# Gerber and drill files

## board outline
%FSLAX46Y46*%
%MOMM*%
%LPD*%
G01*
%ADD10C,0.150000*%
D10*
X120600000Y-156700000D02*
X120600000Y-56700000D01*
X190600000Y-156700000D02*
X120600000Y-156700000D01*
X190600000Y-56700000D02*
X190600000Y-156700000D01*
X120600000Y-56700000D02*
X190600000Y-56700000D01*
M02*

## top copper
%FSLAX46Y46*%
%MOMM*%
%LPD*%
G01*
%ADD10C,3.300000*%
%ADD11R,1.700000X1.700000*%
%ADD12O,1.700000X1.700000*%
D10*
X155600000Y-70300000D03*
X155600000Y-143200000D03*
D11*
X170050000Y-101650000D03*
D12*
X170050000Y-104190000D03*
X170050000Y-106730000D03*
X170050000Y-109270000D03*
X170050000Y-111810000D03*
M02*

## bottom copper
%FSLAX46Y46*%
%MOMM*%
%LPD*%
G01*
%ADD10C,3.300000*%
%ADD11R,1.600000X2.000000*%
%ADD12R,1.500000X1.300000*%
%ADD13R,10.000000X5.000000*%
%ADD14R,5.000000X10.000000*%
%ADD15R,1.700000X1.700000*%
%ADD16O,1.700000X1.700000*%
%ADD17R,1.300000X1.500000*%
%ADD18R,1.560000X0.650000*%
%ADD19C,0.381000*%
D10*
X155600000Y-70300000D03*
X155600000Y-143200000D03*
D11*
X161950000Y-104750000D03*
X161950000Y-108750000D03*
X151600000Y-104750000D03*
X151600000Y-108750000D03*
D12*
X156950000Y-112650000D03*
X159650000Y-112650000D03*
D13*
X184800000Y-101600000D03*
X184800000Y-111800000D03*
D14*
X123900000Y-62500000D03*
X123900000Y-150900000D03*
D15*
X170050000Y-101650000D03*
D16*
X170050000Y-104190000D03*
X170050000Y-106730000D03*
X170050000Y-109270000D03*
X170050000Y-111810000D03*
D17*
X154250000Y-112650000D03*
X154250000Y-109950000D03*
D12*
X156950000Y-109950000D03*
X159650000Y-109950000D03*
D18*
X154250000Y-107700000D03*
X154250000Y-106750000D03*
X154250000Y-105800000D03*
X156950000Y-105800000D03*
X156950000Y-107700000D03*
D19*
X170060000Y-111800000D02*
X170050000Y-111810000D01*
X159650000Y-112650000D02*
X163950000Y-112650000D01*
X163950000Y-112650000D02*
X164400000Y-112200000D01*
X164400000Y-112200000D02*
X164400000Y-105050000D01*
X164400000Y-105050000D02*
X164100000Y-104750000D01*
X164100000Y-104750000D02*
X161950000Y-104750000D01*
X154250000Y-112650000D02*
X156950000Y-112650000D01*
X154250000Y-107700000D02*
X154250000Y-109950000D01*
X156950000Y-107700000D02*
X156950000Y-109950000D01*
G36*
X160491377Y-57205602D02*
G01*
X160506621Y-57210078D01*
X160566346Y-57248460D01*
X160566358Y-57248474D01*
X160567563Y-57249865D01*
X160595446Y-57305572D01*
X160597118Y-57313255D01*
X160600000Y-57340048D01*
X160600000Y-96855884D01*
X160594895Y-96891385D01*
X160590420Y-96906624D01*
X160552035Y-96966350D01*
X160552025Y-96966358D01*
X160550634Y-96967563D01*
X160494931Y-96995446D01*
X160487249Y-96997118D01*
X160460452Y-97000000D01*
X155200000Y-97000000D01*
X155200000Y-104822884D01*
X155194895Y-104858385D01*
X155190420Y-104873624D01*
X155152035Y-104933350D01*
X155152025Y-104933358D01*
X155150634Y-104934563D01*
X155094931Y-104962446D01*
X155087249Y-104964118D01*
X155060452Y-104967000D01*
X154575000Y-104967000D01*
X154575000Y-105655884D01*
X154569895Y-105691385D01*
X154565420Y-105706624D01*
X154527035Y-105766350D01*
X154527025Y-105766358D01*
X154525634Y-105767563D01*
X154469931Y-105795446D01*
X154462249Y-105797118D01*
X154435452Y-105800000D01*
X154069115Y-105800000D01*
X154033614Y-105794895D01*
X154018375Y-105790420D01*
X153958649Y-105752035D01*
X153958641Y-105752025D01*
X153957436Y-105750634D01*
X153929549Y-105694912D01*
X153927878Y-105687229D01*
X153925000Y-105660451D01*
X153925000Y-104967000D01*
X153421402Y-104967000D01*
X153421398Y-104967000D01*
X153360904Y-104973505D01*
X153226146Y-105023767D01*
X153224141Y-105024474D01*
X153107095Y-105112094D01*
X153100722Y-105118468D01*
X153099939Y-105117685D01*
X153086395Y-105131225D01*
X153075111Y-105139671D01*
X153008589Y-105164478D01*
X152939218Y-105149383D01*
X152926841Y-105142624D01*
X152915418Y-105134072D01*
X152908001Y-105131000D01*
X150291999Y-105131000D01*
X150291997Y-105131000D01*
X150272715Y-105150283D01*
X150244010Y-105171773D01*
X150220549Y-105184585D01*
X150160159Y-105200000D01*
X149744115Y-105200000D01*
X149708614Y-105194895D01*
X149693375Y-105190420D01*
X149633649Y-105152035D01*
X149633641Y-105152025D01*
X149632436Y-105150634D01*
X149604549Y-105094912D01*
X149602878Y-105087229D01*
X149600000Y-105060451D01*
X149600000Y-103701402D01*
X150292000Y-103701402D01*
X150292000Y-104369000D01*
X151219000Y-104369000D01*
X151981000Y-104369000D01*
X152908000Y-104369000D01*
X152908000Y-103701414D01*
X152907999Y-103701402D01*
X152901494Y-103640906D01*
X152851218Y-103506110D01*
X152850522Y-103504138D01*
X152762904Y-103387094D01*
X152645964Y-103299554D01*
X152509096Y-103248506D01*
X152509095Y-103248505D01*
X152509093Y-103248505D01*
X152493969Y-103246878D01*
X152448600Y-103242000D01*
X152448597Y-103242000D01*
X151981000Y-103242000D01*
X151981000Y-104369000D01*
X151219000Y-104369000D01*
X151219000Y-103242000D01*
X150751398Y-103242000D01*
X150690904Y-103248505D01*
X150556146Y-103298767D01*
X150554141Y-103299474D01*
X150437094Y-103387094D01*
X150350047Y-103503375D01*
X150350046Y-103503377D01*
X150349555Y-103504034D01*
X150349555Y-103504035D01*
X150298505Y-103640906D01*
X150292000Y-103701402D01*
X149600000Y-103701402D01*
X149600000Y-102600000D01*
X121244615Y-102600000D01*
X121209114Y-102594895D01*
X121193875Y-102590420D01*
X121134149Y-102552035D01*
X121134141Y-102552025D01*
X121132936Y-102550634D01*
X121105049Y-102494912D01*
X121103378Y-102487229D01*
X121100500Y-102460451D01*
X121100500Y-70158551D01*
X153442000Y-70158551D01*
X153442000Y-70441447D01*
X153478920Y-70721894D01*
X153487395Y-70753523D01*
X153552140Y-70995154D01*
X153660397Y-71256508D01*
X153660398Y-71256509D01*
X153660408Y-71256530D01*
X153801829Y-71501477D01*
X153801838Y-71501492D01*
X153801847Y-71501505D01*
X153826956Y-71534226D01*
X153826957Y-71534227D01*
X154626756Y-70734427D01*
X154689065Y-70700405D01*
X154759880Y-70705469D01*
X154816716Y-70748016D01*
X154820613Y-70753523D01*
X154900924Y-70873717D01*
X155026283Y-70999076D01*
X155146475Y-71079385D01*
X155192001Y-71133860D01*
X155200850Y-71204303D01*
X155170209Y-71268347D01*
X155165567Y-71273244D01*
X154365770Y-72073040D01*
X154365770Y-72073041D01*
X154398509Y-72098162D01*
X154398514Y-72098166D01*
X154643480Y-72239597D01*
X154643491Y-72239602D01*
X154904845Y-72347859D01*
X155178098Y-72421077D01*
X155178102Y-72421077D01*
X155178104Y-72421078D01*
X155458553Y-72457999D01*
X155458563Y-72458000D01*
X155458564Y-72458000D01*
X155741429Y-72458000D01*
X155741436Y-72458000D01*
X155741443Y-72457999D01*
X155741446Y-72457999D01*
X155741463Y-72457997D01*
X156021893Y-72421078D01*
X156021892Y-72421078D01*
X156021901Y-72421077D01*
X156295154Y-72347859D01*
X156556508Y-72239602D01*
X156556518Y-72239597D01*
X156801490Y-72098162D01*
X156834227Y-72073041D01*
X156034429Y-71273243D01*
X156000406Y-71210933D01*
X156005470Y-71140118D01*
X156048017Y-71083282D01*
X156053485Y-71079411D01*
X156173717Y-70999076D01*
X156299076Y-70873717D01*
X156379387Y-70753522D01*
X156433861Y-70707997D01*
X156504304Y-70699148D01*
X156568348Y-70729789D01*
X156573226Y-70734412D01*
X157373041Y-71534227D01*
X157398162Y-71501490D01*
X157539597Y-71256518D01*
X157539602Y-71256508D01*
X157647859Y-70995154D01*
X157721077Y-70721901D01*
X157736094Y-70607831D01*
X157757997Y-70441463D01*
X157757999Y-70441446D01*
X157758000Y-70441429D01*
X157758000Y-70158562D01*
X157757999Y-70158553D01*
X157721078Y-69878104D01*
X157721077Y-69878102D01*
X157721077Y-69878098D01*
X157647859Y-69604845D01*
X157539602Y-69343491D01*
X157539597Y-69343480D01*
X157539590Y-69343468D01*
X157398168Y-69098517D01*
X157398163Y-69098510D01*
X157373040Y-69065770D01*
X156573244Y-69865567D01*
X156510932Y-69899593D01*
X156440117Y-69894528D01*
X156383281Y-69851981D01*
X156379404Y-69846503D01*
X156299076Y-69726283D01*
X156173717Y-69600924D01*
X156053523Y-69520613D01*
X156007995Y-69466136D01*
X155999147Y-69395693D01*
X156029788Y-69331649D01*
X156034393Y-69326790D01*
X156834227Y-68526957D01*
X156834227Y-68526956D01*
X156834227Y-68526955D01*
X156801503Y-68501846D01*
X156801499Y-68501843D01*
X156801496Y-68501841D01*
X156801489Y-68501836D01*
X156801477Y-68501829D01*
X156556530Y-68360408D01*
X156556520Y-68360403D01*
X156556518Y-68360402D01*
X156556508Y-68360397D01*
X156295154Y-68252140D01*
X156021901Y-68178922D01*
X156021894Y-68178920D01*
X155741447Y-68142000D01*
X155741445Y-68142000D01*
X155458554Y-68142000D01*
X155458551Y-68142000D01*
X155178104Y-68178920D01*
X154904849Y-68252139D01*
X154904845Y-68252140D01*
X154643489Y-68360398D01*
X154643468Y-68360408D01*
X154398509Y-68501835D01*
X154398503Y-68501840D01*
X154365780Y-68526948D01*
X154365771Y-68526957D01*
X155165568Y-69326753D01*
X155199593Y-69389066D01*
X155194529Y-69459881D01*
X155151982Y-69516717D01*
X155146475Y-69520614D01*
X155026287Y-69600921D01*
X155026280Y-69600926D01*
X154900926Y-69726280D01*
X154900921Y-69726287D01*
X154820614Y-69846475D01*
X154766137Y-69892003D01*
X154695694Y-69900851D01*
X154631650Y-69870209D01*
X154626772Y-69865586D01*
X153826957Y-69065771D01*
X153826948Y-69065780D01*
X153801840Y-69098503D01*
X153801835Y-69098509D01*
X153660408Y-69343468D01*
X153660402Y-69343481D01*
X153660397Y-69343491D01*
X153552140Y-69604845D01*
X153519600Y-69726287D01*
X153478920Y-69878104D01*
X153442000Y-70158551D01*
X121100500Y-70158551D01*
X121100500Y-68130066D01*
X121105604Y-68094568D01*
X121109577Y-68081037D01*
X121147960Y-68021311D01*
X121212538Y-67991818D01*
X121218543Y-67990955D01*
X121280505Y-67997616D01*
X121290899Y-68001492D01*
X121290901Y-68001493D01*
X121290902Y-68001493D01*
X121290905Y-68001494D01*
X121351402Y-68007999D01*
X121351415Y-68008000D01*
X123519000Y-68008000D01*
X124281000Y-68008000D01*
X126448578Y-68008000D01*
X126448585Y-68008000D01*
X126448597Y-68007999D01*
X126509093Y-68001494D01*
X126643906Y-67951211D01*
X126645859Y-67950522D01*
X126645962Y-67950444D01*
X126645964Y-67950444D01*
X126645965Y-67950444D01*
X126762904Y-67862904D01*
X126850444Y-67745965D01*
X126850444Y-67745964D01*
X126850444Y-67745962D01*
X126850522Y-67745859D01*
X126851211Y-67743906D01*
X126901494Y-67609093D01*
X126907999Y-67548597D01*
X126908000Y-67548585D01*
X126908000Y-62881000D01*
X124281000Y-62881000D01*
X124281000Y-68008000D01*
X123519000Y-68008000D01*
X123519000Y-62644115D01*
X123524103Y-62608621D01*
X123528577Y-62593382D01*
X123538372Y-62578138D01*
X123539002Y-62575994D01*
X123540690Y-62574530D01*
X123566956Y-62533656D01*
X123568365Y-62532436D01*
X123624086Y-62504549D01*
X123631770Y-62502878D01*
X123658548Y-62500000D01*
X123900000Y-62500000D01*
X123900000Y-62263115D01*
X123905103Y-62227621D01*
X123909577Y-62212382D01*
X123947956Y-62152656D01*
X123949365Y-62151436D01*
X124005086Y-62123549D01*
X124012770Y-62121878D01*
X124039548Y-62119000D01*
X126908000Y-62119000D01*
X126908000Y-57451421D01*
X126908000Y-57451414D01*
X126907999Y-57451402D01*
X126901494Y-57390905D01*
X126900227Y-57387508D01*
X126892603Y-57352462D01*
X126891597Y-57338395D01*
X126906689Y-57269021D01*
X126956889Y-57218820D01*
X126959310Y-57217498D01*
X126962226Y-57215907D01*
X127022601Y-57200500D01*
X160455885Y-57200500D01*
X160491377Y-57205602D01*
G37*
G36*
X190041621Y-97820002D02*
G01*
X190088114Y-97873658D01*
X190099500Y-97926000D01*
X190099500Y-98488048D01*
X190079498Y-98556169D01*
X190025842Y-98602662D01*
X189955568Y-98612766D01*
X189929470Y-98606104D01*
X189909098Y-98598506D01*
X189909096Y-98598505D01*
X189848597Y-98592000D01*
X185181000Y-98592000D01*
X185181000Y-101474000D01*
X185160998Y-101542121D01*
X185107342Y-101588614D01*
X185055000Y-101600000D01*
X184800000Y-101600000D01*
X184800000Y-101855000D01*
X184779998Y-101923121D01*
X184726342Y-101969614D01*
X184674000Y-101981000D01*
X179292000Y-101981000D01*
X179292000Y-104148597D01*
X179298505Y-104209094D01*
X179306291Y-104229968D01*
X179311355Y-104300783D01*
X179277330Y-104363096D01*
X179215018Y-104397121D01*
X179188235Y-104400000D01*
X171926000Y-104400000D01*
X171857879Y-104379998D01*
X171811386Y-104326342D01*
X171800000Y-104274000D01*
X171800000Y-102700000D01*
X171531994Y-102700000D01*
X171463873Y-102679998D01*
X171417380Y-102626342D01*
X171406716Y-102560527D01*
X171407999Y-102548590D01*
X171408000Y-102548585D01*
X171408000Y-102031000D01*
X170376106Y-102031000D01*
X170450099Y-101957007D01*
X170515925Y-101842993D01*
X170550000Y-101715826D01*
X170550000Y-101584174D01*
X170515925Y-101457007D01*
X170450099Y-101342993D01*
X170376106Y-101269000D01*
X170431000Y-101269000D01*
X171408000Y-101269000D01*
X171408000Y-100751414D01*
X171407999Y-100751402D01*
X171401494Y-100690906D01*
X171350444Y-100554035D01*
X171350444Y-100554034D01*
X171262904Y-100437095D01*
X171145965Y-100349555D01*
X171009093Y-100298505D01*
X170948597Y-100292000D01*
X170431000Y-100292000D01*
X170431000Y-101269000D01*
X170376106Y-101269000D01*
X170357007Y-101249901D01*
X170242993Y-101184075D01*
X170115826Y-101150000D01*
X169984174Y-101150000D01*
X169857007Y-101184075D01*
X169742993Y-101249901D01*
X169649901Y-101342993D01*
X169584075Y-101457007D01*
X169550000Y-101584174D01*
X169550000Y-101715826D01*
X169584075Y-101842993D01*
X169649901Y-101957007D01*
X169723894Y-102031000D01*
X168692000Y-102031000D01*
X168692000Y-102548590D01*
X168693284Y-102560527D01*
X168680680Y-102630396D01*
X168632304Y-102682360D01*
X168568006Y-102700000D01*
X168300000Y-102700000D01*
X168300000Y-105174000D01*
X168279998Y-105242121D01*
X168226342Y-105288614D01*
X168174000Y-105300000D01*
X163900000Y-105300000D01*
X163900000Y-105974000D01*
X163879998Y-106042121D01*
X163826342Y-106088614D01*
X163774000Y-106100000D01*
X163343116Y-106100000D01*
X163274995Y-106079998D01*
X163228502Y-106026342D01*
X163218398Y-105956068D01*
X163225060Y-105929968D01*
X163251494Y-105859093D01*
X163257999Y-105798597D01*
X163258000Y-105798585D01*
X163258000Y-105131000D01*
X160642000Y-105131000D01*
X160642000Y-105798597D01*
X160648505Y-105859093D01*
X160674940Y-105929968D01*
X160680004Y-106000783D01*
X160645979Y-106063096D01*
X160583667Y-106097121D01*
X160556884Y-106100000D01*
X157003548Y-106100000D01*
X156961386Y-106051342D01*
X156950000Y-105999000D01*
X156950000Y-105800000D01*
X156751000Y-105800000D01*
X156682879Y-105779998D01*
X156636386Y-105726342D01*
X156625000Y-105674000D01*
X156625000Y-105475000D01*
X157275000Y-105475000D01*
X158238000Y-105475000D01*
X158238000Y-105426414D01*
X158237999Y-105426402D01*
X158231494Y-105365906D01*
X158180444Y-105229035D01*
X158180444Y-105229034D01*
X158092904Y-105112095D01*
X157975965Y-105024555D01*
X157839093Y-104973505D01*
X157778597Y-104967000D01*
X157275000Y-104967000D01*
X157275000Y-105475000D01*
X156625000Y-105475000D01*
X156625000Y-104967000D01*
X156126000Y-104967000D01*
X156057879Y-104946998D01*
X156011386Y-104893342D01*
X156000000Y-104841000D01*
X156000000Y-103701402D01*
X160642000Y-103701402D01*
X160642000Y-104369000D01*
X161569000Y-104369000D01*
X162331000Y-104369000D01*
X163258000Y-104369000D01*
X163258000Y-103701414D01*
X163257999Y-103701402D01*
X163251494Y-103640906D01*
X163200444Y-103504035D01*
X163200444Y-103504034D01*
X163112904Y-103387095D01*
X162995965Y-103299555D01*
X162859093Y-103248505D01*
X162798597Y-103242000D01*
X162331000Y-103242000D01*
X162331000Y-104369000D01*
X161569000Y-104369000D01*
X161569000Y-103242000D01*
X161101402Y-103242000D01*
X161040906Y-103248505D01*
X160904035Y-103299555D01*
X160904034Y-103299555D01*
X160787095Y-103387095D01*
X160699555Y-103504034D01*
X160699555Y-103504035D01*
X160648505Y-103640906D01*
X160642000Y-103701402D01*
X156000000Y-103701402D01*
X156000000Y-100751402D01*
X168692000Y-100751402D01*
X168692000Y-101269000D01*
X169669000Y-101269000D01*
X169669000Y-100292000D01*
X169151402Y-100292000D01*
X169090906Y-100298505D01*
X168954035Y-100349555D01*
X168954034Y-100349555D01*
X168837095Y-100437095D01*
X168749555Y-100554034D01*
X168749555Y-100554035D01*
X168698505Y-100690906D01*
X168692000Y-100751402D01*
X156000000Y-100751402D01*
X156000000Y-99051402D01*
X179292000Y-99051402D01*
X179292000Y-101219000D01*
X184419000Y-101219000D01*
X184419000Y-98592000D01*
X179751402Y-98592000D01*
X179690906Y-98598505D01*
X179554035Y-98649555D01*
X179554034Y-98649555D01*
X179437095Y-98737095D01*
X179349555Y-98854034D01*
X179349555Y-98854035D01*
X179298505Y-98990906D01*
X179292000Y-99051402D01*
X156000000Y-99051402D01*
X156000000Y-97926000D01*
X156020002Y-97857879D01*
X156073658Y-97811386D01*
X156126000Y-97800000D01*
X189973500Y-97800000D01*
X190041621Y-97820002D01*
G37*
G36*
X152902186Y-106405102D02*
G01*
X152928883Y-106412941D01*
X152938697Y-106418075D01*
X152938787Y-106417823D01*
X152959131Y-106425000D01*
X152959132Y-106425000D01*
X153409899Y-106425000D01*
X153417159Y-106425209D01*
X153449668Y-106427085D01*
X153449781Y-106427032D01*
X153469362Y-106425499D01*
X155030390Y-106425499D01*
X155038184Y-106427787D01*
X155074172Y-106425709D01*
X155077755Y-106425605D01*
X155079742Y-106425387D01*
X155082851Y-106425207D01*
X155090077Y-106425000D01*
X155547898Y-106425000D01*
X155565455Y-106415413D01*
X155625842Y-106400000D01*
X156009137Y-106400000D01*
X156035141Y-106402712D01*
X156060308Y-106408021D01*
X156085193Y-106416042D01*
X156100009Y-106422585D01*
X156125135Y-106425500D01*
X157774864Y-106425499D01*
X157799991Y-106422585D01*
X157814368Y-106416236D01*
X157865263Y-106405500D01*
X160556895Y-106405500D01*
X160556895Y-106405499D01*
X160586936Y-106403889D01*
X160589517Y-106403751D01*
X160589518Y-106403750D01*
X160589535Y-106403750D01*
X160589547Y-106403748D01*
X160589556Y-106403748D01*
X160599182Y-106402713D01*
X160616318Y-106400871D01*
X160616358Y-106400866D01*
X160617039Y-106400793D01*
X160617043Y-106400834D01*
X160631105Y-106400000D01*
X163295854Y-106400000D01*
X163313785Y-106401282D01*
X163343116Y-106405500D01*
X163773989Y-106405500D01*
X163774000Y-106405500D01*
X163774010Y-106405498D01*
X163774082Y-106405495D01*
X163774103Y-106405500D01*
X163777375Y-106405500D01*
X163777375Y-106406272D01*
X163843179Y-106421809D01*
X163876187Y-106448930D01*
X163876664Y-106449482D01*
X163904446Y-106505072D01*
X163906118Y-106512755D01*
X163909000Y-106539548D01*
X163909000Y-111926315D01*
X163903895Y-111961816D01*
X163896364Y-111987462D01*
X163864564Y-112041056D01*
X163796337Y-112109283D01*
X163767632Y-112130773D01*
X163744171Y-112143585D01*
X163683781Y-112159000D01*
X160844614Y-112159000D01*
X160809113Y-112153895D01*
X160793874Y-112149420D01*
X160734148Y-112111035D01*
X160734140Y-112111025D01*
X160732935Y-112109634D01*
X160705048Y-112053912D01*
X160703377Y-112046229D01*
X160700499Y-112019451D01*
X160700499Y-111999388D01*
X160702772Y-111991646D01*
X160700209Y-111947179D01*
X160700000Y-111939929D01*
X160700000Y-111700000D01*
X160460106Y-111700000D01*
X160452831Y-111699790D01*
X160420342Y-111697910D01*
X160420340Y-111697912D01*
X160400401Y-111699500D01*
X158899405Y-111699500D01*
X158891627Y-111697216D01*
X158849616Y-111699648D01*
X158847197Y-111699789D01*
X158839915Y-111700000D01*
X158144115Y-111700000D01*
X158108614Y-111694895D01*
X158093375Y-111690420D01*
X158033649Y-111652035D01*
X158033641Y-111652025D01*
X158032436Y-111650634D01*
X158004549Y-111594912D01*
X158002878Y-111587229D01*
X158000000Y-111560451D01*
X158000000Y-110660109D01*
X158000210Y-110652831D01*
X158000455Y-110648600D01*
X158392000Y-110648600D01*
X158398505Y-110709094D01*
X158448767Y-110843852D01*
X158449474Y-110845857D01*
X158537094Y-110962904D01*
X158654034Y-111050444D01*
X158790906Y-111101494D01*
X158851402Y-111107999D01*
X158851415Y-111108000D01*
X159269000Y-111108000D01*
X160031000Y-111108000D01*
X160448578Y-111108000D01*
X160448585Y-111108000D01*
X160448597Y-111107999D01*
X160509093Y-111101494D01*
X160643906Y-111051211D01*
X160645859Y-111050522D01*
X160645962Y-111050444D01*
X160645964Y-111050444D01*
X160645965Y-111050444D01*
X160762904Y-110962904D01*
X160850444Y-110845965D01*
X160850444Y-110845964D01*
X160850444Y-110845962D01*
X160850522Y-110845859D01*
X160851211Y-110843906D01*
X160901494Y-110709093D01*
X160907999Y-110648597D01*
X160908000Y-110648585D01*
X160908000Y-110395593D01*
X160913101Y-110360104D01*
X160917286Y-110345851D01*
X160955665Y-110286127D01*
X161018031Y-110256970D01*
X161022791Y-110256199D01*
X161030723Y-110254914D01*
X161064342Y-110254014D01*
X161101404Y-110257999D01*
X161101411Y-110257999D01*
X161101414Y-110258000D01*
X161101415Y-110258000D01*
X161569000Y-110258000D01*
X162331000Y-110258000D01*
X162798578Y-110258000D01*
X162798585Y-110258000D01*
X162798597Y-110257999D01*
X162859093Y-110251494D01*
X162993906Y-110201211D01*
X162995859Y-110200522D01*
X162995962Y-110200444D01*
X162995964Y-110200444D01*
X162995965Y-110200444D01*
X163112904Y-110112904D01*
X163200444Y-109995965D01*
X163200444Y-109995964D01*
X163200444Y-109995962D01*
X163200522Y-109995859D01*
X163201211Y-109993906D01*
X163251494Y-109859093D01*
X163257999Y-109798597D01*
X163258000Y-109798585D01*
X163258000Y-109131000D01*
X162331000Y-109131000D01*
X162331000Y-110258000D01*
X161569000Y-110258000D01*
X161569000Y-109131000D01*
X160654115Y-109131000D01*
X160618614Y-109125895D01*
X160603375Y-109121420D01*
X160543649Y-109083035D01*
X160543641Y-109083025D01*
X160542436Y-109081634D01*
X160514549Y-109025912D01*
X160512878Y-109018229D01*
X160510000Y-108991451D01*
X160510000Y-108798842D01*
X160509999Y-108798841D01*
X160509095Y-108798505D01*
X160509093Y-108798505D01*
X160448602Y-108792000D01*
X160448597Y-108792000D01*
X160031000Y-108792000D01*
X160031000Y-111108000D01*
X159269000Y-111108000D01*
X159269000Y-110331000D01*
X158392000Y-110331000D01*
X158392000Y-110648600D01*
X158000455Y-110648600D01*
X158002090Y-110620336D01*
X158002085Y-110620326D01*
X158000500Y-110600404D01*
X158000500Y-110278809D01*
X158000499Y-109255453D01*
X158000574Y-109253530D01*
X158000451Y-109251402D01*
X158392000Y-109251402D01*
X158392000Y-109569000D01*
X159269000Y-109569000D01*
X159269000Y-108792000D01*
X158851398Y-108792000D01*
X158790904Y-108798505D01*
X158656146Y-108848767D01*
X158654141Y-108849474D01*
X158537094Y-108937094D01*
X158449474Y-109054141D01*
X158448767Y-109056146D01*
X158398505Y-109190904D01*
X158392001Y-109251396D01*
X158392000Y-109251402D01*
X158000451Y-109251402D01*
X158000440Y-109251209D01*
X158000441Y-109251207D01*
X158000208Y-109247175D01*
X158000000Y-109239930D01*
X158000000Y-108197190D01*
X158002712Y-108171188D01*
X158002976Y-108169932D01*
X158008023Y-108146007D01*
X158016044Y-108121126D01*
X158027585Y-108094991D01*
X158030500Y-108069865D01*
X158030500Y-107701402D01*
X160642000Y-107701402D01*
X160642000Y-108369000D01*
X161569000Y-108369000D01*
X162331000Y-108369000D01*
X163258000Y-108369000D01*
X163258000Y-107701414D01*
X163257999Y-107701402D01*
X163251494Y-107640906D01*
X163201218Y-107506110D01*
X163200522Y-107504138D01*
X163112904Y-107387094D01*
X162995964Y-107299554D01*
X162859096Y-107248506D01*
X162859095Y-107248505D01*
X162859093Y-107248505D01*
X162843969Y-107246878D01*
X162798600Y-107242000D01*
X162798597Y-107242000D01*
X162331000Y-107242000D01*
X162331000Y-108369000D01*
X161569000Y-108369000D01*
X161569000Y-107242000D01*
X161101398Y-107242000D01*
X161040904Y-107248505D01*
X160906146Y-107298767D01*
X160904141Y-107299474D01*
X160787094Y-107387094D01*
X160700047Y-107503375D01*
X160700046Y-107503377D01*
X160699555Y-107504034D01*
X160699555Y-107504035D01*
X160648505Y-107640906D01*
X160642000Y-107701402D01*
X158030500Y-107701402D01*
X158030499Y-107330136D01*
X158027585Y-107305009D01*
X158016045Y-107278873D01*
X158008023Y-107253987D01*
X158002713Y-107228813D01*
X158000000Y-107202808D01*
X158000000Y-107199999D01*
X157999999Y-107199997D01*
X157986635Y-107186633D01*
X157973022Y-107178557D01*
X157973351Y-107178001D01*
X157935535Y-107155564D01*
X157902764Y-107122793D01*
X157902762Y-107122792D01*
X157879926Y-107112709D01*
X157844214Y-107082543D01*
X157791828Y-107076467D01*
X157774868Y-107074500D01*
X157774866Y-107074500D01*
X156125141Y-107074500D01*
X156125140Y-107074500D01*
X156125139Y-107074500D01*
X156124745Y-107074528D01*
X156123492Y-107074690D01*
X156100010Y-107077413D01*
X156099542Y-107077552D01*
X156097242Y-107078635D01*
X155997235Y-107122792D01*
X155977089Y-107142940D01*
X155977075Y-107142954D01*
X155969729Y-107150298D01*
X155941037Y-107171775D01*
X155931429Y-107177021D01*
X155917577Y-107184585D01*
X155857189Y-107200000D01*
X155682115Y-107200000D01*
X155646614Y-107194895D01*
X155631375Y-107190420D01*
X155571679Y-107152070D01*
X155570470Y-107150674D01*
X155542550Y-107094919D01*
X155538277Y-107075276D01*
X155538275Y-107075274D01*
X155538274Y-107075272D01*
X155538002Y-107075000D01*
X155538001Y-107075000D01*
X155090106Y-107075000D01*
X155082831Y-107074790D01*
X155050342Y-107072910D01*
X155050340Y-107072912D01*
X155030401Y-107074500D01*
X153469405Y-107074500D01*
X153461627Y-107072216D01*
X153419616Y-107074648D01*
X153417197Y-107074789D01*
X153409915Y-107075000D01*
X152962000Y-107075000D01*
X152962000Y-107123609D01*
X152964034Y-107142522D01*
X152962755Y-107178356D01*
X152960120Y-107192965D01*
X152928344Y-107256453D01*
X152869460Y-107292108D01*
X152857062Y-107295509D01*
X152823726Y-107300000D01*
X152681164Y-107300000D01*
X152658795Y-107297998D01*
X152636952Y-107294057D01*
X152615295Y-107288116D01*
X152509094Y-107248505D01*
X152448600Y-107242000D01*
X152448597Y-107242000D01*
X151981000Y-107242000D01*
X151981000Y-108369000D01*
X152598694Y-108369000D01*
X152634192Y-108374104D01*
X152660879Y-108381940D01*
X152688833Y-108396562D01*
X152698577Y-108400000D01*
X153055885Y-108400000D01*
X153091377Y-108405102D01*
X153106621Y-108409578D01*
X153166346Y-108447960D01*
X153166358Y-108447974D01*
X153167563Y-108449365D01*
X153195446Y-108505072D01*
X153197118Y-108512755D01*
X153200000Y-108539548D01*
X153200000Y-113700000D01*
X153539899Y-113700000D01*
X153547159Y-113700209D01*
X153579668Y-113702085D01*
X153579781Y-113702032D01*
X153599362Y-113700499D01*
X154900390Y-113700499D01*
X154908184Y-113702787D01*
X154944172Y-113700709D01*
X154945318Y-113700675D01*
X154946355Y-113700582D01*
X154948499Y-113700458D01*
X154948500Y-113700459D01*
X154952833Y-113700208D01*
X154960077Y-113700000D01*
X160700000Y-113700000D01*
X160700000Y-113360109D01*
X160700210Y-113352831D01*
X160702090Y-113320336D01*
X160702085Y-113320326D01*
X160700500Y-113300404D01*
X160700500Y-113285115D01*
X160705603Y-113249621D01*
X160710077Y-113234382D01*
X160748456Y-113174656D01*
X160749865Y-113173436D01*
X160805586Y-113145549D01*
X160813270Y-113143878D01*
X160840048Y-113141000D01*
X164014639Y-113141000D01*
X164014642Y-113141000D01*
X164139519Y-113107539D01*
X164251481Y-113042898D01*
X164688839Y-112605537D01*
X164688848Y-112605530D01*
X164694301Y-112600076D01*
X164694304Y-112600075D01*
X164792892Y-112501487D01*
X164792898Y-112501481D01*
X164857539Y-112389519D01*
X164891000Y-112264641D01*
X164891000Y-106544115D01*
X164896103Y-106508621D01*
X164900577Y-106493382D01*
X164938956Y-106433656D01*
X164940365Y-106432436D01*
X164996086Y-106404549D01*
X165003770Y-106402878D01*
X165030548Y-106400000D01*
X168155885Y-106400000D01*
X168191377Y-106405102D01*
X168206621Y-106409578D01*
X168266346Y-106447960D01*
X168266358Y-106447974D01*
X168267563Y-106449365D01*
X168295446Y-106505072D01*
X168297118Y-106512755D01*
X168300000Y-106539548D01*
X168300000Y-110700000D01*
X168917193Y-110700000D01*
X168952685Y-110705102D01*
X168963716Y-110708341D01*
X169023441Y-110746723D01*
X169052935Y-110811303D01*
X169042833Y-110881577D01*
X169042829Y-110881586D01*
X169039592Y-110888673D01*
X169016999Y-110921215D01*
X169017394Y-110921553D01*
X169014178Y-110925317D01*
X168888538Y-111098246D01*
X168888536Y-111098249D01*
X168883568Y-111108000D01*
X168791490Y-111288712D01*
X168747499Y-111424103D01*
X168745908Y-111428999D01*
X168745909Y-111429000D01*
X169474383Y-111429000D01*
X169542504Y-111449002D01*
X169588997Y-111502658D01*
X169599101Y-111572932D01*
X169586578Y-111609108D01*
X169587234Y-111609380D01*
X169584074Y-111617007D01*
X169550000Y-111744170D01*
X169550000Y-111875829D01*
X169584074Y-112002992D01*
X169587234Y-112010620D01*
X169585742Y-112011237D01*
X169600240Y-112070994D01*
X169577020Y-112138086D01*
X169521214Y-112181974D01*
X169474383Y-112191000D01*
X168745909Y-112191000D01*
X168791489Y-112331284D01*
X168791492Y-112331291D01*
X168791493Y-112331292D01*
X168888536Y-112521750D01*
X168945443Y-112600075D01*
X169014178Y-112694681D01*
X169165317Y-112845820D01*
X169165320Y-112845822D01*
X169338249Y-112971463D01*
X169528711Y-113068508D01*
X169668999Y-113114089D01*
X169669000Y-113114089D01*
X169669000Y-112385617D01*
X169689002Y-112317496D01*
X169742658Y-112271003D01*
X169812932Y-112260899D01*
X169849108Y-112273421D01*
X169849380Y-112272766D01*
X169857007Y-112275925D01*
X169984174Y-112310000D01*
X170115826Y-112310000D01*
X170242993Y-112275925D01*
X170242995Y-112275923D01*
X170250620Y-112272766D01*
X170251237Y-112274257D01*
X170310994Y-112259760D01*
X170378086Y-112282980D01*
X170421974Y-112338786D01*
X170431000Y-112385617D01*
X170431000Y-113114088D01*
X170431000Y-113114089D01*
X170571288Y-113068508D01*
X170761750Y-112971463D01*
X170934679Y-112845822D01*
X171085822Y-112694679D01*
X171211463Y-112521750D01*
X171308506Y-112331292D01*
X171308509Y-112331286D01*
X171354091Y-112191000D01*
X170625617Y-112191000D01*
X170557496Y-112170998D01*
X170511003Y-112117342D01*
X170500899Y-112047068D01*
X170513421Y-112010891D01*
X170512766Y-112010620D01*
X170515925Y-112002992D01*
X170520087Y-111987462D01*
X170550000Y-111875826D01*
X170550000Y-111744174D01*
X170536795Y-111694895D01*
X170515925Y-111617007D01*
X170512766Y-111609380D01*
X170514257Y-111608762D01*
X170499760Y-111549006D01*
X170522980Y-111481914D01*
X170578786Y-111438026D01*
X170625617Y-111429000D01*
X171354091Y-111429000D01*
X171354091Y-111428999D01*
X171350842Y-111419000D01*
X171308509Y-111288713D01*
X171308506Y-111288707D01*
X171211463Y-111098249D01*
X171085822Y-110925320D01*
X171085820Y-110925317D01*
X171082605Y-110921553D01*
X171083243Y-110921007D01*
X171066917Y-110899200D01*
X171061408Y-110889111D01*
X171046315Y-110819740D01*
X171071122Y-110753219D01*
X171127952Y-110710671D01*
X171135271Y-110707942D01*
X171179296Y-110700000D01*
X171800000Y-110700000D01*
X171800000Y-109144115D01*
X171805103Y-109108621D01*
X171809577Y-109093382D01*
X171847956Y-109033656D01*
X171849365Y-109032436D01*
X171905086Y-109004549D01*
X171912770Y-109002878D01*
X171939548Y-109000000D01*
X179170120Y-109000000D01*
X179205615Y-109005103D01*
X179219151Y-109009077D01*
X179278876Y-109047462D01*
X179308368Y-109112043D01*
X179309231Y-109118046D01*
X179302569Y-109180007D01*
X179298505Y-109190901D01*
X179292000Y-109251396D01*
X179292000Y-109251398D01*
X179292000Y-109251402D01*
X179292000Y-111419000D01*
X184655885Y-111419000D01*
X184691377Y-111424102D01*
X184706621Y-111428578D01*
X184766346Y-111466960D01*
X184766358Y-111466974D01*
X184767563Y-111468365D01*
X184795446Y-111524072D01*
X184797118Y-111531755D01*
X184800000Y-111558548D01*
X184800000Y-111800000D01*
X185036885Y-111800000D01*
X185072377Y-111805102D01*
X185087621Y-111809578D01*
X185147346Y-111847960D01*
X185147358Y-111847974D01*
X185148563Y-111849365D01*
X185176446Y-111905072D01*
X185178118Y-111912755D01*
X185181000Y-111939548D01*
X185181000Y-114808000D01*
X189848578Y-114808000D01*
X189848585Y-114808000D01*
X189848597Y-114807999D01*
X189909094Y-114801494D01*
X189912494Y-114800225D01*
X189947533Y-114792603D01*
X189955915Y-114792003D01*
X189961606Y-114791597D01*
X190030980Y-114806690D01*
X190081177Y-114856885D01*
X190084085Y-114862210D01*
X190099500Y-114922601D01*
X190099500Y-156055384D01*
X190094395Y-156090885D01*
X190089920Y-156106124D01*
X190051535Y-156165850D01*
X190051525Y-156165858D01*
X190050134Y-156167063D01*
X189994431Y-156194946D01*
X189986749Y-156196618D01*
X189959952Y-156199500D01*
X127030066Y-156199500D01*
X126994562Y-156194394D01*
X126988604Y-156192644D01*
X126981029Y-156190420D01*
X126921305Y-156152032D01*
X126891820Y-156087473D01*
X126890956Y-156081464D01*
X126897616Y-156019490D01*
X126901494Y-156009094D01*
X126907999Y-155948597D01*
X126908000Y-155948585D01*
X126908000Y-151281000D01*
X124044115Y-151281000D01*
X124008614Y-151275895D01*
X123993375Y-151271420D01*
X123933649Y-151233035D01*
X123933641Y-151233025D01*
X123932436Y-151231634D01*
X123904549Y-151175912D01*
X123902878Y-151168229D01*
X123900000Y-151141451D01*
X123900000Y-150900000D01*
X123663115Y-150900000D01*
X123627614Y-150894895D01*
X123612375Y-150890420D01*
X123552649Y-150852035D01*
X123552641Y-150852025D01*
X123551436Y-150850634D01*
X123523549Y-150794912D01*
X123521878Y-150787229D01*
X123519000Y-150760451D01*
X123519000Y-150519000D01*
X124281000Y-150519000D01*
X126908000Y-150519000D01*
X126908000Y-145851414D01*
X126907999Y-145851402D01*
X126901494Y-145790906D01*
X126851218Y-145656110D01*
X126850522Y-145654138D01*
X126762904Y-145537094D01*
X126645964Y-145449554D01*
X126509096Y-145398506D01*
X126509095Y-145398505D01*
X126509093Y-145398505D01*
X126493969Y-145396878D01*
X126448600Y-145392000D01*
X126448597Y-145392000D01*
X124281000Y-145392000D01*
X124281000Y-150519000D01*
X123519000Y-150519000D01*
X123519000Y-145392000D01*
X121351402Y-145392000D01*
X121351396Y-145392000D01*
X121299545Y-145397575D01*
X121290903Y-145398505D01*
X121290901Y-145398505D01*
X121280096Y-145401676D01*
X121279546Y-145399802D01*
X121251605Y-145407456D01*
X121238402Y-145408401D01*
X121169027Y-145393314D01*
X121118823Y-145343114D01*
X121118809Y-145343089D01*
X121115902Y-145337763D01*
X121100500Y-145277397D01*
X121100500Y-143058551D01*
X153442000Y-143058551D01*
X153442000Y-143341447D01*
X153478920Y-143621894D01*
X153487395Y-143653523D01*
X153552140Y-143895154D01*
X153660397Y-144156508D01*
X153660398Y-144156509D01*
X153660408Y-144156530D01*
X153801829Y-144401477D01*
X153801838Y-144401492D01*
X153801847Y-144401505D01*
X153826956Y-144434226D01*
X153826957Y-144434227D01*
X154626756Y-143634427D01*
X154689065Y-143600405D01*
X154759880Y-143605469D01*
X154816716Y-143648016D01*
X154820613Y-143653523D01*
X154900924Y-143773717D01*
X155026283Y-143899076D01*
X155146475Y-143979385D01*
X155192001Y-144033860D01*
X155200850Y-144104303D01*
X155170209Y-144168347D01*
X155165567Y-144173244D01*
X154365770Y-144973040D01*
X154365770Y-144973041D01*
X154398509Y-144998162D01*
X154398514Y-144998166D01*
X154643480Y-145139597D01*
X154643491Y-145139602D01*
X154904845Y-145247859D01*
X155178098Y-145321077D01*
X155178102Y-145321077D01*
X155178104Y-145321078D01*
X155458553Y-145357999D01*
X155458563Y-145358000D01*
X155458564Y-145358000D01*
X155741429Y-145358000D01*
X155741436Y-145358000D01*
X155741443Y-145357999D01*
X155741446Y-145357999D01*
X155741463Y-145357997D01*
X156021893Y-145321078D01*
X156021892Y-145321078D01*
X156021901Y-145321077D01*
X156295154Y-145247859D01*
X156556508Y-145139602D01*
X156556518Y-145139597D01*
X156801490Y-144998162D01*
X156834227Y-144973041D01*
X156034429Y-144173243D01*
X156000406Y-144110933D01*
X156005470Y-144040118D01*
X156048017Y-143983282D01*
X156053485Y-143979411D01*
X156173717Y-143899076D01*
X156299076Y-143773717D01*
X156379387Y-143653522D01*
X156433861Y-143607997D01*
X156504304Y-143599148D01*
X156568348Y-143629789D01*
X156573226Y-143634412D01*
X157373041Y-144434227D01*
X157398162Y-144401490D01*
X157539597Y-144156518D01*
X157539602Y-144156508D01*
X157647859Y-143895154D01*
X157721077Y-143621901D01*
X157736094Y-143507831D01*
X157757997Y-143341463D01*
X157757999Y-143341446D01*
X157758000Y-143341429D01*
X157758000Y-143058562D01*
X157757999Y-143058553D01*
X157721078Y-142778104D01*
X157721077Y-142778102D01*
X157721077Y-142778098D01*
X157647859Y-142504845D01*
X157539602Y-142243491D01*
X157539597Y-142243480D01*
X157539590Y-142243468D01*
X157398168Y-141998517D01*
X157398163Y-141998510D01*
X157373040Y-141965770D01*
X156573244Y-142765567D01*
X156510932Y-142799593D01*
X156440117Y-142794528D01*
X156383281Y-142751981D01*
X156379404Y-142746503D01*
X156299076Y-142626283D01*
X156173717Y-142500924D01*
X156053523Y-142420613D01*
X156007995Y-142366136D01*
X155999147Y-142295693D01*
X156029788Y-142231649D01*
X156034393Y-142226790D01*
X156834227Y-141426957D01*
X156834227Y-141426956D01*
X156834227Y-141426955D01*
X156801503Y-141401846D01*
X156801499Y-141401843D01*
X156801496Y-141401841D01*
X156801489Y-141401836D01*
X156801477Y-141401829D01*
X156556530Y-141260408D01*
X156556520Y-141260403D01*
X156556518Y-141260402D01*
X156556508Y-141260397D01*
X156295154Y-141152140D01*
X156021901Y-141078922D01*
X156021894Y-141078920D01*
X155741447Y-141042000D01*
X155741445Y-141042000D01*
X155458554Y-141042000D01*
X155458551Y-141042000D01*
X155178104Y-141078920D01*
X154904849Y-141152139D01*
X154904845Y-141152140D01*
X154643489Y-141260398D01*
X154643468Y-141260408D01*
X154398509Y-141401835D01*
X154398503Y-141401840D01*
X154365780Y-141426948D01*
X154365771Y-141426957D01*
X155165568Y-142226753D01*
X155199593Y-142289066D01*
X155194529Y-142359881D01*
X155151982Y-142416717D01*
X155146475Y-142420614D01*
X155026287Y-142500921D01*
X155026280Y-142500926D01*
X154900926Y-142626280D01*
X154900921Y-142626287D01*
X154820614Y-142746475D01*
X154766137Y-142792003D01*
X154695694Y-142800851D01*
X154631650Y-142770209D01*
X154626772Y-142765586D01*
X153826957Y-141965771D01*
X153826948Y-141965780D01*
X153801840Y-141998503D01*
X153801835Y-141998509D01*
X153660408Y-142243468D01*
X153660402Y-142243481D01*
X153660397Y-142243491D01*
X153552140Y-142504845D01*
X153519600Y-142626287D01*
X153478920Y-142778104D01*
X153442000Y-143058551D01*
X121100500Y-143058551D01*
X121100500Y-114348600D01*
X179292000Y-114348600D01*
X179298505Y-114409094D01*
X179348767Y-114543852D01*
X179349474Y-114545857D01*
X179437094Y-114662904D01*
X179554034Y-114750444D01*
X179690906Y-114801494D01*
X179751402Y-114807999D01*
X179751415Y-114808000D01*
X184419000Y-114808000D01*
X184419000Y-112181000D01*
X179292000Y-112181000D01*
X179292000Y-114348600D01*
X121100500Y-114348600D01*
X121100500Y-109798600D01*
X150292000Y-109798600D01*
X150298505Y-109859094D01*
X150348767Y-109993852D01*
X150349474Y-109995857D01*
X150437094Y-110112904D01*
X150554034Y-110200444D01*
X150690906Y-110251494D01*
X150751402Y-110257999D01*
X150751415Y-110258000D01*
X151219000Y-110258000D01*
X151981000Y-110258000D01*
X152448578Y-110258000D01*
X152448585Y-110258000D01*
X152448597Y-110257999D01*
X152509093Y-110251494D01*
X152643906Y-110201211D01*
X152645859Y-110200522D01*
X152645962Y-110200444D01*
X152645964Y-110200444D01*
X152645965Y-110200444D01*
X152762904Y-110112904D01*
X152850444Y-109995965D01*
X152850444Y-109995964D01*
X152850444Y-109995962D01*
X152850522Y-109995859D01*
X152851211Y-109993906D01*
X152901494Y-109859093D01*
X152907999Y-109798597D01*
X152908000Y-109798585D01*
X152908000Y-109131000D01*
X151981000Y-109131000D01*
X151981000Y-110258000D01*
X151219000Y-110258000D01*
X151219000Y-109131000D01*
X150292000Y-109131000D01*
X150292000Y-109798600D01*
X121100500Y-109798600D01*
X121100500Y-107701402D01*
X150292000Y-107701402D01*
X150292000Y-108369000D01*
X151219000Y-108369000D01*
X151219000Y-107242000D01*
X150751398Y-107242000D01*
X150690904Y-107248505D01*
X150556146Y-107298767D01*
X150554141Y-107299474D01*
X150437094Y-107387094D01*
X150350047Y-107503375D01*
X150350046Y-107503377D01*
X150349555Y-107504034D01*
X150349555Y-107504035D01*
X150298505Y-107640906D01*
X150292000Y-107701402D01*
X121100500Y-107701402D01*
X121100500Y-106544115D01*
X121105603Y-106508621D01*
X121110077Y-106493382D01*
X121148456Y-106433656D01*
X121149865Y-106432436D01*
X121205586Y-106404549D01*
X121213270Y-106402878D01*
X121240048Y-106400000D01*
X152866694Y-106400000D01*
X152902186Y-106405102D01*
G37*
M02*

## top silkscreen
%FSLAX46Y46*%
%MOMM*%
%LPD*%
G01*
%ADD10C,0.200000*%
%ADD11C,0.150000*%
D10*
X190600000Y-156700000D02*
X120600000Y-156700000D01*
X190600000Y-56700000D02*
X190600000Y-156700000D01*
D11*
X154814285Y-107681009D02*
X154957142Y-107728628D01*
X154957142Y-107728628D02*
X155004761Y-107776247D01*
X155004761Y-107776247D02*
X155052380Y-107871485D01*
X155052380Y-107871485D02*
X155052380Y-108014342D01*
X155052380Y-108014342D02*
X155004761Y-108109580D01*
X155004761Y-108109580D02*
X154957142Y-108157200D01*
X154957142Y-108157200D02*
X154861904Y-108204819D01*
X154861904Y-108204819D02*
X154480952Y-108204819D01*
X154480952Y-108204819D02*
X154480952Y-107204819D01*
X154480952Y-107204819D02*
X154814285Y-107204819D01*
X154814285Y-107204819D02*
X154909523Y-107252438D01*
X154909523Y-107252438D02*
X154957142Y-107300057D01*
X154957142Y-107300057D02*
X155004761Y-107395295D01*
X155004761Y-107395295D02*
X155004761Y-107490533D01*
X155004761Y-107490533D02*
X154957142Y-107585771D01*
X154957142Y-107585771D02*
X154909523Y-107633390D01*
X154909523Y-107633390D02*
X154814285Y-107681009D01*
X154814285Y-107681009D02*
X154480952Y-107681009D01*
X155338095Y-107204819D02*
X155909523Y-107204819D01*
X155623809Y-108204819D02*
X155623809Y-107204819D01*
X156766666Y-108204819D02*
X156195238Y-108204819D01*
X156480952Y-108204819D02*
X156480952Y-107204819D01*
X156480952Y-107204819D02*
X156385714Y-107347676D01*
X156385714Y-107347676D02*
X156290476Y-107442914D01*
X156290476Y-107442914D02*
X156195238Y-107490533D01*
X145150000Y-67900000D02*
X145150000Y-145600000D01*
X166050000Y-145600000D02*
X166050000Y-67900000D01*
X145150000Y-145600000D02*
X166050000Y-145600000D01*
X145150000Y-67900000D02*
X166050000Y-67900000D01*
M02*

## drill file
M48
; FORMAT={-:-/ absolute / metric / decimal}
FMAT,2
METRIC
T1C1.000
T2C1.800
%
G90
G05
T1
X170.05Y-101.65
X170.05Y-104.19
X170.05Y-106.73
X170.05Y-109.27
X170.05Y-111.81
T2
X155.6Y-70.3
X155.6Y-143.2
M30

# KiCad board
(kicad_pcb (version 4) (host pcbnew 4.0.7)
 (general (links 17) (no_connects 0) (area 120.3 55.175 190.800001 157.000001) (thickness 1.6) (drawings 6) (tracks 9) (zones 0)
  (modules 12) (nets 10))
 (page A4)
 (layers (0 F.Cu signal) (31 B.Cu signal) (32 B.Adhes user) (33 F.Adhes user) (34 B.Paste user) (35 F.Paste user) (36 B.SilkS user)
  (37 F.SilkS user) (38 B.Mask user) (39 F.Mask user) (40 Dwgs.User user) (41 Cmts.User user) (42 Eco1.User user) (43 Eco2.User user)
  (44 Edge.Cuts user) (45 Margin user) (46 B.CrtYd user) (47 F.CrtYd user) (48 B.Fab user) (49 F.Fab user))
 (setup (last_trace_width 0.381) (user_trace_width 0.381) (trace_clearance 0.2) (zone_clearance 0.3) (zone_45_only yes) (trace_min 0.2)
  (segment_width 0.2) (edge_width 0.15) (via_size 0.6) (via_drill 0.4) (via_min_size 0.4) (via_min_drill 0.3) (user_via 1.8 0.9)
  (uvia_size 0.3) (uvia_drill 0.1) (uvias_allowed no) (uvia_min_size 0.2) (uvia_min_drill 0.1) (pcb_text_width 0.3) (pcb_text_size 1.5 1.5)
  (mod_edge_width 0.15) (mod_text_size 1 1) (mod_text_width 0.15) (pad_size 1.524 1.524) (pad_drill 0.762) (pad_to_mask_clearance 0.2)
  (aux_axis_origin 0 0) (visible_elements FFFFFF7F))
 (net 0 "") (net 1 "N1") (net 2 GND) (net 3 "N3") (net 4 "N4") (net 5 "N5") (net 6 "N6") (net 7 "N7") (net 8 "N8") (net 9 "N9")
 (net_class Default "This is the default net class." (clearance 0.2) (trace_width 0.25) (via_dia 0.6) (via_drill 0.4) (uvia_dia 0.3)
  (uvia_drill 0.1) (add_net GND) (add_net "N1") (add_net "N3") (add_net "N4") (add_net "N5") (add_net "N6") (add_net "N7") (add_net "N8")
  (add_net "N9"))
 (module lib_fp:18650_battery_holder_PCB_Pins (layer F.Cu) (at 155.6 106.75)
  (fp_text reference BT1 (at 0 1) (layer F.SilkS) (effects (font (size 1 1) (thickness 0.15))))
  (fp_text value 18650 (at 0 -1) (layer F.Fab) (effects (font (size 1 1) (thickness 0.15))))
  (fp_line (start -10.45 -38.85) (end -10.45 38.85) (layer F.SilkS) (width 0.15))
  (fp_line (start 10.45 38.85) (end 10.45 -38.85) (layer F.SilkS) (width 0.15))
  (fp_line (start -10.45 38.85) (end 10.45 38.85) (layer F.SilkS) (width 0.15))
  (fp_line (start -10.45 -38.85) (end 10.45 -38.85) (layer F.SilkS) (width 0.15))
  (pad 1 thru_hole circle (at 0 -36.45) (size 3.3 3.3) (drill 1.8) (layers *.Cu *.Mask) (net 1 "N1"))
  (pad 2 thru_hole circle (at 0 36.45) (size 3.3 3.3) (drill 1.8) (layers *.Cu *.Mask) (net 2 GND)))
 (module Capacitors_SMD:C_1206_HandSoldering (layer B.Cu) (at 161.95 106.75 270)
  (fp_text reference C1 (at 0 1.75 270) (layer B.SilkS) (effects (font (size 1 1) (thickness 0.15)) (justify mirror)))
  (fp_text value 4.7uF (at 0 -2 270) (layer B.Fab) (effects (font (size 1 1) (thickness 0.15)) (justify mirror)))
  (pad 1 smd rect (at -2 0 270) (size 2 1.6) (layers B.Cu B.Paste B.Mask) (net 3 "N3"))
  (pad 2 smd rect (at 2 0 270) (size 2 1.6) (layers B.Cu B.Paste B.Mask) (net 2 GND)))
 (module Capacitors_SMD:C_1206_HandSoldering (layer B.Cu) (at 151.6 106.75 270)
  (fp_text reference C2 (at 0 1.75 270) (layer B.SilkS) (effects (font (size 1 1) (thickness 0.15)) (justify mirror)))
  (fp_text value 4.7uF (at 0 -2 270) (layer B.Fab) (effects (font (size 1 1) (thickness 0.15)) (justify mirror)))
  (pad 1 smd rect (at -2 0 270) (size 2 1.6) (layers B.Cu B.Paste B.Mask) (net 1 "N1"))
  (pad 2 smd rect (at 2 0 270) (size 2 1.6) (layers B.Cu B.Paste B.Mask) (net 2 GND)))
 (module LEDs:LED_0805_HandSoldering (layer B.Cu) (at 158.3 112.65)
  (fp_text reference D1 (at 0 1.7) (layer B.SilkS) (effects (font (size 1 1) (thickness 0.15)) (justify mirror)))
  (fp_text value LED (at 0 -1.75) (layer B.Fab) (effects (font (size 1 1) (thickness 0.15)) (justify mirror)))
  (pad 1 smd rect (at -1.35 0) (size 1.5 1.3) (layers B.Cu B.Paste B.Mask) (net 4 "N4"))
  (pad 2 smd rect (at 1.35 0) (size 1.5 1.3) (layers B.Cu B.Paste B.Mask) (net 3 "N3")))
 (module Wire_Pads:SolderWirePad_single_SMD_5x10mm (layer B.Cu) (at 184.8 101.6 90)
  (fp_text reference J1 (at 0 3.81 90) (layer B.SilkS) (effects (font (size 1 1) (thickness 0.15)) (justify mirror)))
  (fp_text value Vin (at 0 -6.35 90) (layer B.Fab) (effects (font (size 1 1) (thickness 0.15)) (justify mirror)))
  (pad 1 smd rect (at 0 0 90) (size 5 10) (layers B.Cu B.Paste B.Mask) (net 3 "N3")))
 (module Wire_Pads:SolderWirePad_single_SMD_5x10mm (layer B.Cu) (at 184.8 111.8 90)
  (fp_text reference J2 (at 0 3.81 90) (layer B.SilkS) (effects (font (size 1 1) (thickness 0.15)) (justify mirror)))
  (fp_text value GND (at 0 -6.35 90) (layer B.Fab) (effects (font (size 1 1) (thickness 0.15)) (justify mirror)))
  (pad 1 smd rect (at 0 0 90) (size 5 10) (layers B.Cu B.Paste B.Mask) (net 2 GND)))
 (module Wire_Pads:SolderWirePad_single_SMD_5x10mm (layer B.Cu) (at 123.9 62.5)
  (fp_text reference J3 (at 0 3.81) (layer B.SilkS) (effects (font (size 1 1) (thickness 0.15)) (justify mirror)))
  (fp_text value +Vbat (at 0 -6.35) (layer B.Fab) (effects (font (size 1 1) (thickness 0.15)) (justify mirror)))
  (pad 1 smd rect (at 0 0) (size 5 10) (layers B.Cu B.Paste B.Mask) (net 1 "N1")))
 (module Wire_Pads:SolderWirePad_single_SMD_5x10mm (layer B.Cu) (at 123.9 150.9)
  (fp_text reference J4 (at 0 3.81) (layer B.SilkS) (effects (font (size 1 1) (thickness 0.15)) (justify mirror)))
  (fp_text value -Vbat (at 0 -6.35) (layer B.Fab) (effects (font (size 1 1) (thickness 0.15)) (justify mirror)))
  (pad 1 smd rect (at 0 0) (size 5 10) (layers B.Cu B.Paste B.Mask) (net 2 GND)))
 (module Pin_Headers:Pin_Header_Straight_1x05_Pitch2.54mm (layer B.Cu) (at 170.05 101.65 180)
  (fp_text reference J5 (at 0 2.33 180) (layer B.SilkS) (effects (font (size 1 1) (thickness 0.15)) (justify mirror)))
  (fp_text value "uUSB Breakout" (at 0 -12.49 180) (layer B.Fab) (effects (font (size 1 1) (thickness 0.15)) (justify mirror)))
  (pad 1 thru_hole rect (at 0 0 180) (size 1.7 1.7) (drill 1) (layers *.Cu *.Mask) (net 3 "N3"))
  (pad 2 thru_hole oval (at 0 -2.54 180) (size 1.7 1.7) (drill 1) (layers *.Cu *.Mask) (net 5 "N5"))
  (pad 3 thru_hole oval (at 0 -5.08 180) (size 1.7 1.7) (drill 1) (layers *.Cu *.Mask) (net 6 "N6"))
  (pad 4 thru_hole oval (at 0 -7.62 180) (size 1.7 1.7) (drill 1) (layers *.Cu *.Mask) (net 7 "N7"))
  (pad 5 thru_hole oval (at 0 -10.16 180) (size 1.7 1.7) (drill 1) (layers *.Cu *.Mask) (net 2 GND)))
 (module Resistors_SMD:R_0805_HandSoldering (layer B.Cu) (at 154.25 111.3 90)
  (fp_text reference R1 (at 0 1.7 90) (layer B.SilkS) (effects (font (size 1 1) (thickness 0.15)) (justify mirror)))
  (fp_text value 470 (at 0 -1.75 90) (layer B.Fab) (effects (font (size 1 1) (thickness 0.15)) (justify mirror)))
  (pad 1 smd rect (at -1.35 0 90) (size 1.5 1.3) (layers B.Cu B.Paste B.Mask) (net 4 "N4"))
  (pad 2 smd rect (at 1.35 0 90) (size 1.5 1.3) (layers B.Cu B.Paste B.Mask) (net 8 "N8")))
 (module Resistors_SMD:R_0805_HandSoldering (layer B.Cu) (at 158.3 109.95)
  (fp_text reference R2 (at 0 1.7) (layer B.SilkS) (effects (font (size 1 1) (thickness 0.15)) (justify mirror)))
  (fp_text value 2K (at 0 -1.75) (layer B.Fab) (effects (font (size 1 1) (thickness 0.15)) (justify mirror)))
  (pad 1 smd rect (at -1.35 0) (size 1.5 1.3) (layers B.Cu B.Paste B.Mask) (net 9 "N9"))
  (pad 2 smd rect (at 1.35 0) (size 1.5 1.3) (layers B.Cu B.Paste B.Mask) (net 2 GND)))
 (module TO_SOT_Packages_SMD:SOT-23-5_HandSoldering (layer B.Cu) (at 155.6 106.75)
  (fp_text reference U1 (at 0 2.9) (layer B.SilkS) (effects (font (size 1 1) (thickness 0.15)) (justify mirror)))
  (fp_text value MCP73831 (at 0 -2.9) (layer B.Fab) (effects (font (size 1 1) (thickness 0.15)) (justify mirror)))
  (pad 1 smd rect (at -1.35 0.95) (size 1.56 0.65) (layers B.Cu B.Paste B.Mask) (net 8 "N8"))
  (pad 2 smd rect (at -1.35 0) (size 1.56 0.65) (layers B.Cu B.Paste B.Mask) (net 2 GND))
  (pad 3 smd rect (at -1.35 -0.95) (size 1.56 0.65) (layers B.Cu B.Paste B.Mask) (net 1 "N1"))
  (pad 4 smd rect (at 1.35 -0.95) (size 1.56 0.65) (layers B.Cu B.Paste B.Mask) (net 3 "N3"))
  (pad 5 smd rect (at 1.35 0.95) (size 1.56 0.65) (layers B.Cu B.Paste B.Mask) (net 9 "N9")))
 (gr_line (start 190.6 156.7) (end 120.6 156.7) (angle 90) (layer F.SilkS) (width 0.2))
 (gr_line (start 190.6 56.7) (end 190.6 156.7) (angle 90) (layer F.SilkS) (width 0.2))
 (gr_line (start 120.6 156.7) (end 120.6 56.7) (angle 90) (layer Edge.Cuts) (width 0.15))
 (gr_line (start 190.6 156.7) (end 120.6 156.7) (angle 90) (layer Edge.Cuts) (width 0.15))
 (gr_line (start 190.6 56.7) (end 190.6 156.7) (angle 90) (layer Edge.Cuts) (width 0.15))
 (gr_line (start 120.6 56.7) (end 190.6 56.7) (angle 90) (layer Edge.Cuts) (width 0.15))
 (segment (start 170.06 111.8) (end 170.05 111.81) (width 0.381) (layer B.Cu) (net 2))
 (segment (start 159.65 112.65) (end 163.95 112.65) (width 0.381) (layer B.Cu) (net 3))
 (segment (start 163.95 112.65) (end 164.4 112.2) (width 0.381) (layer B.Cu) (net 3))
 (segment (start 164.4 112.2) (end 164.4 105.05) (width 0.381) (layer B.Cu) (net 3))
 (segment (start 164.4 105.05) (end 164.1 104.75) (width 0.381) (layer B.Cu) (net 3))
 (segment (start 164.1 104.75) (end 161.95 104.75) (width 0.381) (layer B.Cu) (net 3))
 (segment (start 154.25 112.65) (end 156.95 112.65) (width 0.381) (layer B.Cu) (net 4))
 (segment (start 154.25 107.7) (end 154.25 109.95) (width 0.381) (layer B.Cu) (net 8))
 (segment (start 156.95 107.7) (end 156.95 109.95) (width 0.381) (layer B.Cu) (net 9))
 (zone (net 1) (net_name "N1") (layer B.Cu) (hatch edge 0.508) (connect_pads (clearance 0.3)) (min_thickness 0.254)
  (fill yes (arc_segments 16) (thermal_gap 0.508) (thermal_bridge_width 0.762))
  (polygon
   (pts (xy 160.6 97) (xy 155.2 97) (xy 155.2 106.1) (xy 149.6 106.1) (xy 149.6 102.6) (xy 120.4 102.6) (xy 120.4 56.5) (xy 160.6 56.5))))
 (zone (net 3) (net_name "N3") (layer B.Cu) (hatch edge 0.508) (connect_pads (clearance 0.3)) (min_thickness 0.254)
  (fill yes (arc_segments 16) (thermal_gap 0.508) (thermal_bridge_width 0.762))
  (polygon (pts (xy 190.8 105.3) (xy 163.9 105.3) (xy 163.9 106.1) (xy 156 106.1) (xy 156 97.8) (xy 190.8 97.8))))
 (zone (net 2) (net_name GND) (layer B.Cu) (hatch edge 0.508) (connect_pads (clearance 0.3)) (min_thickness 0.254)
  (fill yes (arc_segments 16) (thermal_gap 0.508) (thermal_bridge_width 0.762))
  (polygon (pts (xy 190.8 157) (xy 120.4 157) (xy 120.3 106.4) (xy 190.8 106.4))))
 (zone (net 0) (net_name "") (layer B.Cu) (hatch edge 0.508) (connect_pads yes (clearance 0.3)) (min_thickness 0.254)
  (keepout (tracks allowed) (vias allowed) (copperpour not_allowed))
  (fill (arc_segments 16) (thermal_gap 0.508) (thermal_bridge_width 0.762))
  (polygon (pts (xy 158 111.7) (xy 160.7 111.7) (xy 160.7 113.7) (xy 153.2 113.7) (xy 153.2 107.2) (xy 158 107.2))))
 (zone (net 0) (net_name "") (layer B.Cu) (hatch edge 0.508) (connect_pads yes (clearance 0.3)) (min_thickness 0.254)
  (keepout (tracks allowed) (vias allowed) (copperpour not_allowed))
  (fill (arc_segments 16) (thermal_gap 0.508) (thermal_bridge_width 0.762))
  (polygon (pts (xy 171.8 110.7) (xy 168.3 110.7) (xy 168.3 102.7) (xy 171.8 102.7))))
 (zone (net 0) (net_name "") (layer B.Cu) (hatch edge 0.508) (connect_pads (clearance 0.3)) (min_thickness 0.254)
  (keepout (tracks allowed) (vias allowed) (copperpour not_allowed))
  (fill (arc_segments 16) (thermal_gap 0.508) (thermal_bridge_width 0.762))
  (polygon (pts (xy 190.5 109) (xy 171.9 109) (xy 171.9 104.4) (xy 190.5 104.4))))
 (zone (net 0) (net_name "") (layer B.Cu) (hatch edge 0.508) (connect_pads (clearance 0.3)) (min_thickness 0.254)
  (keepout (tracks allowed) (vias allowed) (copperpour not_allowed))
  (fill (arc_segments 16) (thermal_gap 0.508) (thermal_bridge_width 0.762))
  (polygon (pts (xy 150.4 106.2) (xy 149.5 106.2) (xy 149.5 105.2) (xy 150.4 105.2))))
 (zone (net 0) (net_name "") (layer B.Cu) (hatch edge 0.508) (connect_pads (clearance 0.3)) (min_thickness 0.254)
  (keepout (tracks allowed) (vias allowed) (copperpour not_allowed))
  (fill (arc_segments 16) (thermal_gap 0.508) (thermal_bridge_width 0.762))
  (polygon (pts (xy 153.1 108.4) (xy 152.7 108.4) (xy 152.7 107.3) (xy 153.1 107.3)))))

